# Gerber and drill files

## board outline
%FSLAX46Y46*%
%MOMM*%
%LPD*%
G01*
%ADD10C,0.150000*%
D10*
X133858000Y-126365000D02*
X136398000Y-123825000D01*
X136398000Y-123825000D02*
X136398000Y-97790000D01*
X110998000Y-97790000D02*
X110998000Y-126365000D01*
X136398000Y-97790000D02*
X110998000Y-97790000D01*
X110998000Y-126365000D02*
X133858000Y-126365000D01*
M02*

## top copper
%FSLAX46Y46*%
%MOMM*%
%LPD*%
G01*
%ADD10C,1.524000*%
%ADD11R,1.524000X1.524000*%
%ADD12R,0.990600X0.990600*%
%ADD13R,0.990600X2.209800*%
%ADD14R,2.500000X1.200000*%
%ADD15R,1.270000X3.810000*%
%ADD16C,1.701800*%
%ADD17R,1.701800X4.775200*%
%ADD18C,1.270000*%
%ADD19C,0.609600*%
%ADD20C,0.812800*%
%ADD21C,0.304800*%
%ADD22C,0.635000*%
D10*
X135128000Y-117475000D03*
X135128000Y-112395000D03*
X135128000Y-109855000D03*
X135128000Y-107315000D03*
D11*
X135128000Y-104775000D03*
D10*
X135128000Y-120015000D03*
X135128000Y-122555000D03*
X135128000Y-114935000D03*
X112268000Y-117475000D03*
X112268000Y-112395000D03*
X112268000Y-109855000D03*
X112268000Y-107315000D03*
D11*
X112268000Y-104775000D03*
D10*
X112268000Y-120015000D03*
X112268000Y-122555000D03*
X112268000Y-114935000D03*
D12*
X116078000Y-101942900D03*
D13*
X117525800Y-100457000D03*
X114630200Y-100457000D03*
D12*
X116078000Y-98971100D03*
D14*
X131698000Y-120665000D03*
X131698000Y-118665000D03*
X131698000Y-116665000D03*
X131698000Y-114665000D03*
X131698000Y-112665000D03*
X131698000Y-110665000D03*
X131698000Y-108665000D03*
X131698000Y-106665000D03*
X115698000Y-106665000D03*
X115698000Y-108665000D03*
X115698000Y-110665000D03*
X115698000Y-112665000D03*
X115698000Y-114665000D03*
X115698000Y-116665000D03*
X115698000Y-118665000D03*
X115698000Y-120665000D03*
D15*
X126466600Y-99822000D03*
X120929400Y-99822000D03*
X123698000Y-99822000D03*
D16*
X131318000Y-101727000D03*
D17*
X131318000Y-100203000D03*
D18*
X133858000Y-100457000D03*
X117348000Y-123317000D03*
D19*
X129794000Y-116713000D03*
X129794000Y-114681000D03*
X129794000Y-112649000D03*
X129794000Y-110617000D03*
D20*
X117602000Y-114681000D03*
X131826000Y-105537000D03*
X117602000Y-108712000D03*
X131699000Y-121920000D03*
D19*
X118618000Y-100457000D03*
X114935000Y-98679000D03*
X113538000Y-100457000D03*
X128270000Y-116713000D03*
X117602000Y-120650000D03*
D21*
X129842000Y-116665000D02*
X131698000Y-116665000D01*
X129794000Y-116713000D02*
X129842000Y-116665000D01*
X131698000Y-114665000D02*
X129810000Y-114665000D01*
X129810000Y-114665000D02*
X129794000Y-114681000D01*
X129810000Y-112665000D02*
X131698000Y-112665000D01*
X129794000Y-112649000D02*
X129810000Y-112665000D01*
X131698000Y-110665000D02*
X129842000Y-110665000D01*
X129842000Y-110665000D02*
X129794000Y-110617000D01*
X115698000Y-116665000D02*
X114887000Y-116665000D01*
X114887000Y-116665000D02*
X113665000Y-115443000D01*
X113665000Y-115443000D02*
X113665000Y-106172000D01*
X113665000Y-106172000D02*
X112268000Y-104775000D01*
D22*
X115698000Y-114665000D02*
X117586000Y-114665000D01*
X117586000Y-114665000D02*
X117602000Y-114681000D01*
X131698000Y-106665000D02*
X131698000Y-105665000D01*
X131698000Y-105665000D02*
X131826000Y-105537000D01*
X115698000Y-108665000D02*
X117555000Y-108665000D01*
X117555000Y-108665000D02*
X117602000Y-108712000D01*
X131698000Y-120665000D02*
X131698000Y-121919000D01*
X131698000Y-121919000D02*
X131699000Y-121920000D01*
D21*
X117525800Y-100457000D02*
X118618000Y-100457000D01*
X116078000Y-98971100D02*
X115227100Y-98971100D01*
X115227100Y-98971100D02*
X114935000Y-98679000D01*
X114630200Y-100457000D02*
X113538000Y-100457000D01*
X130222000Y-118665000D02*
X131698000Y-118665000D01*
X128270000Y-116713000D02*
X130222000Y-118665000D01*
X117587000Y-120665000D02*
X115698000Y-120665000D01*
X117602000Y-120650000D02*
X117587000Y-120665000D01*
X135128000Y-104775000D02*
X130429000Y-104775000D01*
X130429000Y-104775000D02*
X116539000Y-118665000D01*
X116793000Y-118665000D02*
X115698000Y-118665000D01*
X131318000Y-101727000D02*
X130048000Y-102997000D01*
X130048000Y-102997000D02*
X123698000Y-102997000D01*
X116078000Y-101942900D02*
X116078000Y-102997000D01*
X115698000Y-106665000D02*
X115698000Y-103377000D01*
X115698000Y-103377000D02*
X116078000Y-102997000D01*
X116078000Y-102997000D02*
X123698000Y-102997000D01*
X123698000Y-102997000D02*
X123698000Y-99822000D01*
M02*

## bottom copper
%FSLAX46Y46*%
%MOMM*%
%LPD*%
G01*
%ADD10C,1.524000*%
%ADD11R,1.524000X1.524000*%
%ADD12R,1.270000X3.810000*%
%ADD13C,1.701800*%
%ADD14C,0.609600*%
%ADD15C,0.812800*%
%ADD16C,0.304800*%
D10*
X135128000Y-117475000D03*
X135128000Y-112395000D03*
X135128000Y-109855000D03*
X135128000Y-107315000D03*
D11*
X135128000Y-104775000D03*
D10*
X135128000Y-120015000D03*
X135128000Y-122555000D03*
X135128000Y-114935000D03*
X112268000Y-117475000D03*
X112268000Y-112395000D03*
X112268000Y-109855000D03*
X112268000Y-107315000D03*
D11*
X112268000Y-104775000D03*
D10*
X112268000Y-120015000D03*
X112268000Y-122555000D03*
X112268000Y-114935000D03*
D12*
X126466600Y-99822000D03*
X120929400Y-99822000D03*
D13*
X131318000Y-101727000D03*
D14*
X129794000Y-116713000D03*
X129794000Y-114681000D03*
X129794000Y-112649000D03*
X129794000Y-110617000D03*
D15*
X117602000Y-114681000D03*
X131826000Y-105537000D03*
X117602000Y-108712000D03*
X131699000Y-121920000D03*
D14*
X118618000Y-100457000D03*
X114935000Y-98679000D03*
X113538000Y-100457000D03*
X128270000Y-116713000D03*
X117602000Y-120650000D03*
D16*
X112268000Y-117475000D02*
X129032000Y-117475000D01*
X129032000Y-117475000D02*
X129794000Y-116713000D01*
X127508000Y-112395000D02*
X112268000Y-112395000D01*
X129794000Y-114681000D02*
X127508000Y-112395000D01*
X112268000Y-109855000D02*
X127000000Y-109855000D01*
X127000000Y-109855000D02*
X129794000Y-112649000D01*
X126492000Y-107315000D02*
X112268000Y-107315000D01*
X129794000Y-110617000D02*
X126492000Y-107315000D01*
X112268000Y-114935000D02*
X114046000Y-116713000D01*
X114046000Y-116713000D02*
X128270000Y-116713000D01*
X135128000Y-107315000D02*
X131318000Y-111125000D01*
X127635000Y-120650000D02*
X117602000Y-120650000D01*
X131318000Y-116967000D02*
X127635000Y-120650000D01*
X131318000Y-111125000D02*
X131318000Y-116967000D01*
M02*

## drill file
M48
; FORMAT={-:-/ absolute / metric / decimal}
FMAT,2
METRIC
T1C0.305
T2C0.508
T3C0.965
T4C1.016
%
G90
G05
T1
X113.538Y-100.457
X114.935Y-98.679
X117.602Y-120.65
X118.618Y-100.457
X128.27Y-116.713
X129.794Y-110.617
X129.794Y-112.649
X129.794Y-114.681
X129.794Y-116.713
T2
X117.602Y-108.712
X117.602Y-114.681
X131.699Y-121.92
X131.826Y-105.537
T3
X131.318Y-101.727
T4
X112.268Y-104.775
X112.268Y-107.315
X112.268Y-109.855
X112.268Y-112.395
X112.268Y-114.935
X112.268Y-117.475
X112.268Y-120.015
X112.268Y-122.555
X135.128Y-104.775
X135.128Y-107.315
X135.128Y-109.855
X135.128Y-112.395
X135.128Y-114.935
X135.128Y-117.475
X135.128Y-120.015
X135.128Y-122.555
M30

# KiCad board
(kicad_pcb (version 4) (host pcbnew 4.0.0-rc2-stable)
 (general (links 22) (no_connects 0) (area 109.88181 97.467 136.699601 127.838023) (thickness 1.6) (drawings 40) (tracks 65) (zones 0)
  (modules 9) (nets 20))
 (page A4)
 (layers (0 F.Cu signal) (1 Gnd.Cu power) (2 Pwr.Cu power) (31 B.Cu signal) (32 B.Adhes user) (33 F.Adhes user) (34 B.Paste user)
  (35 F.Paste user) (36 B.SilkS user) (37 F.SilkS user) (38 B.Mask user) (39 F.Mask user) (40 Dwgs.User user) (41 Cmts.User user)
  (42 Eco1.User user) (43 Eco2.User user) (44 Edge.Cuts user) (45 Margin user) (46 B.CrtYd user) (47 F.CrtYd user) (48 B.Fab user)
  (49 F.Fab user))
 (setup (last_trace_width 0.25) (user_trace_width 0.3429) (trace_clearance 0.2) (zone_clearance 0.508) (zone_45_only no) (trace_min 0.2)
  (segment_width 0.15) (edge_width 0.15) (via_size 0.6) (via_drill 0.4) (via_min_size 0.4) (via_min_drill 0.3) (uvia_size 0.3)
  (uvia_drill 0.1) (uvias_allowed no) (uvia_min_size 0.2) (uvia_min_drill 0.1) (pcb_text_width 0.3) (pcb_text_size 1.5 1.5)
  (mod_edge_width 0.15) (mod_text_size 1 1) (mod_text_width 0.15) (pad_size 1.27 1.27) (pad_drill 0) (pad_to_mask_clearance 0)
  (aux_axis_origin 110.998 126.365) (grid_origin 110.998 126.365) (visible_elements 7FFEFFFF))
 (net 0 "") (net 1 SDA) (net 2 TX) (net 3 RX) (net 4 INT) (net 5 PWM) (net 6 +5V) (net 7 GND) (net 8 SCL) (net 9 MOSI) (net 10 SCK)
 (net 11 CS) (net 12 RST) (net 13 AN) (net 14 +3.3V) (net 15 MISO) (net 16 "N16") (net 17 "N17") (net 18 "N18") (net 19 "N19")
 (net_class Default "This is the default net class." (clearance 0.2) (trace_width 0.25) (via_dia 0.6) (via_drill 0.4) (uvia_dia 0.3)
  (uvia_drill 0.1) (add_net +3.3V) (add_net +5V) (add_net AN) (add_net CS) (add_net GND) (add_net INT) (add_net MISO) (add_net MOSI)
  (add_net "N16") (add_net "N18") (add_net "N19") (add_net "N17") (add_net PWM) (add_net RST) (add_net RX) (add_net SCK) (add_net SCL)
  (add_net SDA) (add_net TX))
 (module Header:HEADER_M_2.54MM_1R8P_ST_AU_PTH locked (layer B.Cu) (at 135.128 113.665 270)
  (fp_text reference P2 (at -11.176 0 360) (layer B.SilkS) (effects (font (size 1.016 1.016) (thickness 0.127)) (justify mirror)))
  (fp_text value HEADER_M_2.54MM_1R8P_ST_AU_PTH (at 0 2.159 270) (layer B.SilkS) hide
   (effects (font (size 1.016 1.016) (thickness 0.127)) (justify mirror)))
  (pad 6 thru_hole circle (at 3.81 0 270) (size 1.524 1.524) (drill 1.016) (layers *.Cu *.Mask) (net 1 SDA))
  (pad 4 thru_hole circle (at -1.27 0 270) (size 1.524 1.524) (drill 1.016) (layers *.Cu *.Mask) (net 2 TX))
  (pad 3 thru_hole circle (at -3.81 0 270) (size 1.524 1.524) (drill 1.016) (layers *.Cu *.Mask) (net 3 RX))
  (pad 2 thru_hole circle (at -6.35 0 270) (size 1.524 1.524) (drill 1.016) (layers *.Cu *.Mask) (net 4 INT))
  (pad 1 thru_hole rect (at -8.89 0 270) (size 1.524 1.524) (drill 1.016) (layers *.Cu *.Mask) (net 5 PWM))
  (pad 7 thru_hole circle (at 6.35 0 270) (size 1.524 1.524) (drill 1.016) (layers *.Cu *.Mask) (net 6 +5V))
  (pad 8 thru_hole circle (at 8.89 0 270) (size 1.524 1.524) (drill 1.016) (layers *.Cu *.Mask) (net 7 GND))
  (pad 5 thru_hole circle (at 1.27 0 270) (size 1.524 1.524) (drill 1.016) (layers *.Cu *.Mask) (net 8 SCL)))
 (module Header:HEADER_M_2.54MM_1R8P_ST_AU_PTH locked (layer B.Cu) (at 112.268 113.665 270)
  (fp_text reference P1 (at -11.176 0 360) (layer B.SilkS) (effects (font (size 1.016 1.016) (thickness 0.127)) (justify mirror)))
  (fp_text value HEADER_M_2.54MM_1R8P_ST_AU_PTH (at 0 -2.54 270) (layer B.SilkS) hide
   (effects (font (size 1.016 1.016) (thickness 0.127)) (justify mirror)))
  (pad 6 thru_hole circle (at 3.81 0 270) (size 1.524 1.524) (drill 1.016) (layers *.Cu *.Mask) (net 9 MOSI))
  (pad 4 thru_hole circle (at -1.27 0 270) (size 1.524 1.524) (drill 1.016) (layers *.Cu *.Mask) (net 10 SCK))
  (pad 3 thru_hole circle (at -3.81 0 270) (size 1.524 1.524) (drill 1.016) (layers *.Cu *.Mask) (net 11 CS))
  (pad 2 thru_hole circle (at -6.35 0 270) (size 1.524 1.524) (drill 1.016) (layers *.Cu *.Mask) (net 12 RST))
  (pad 1 thru_hole rect (at -8.89 0 270) (size 1.524 1.524) (drill 1.016) (layers *.Cu *.Mask) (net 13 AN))
  (pad 7 thru_hole circle (at 6.35 0 270) (size 1.524 1.524) (drill 1.016) (layers *.Cu *.Mask) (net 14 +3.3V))
  (pad 8 thru_hole circle (at 8.89 0 270) (size 1.524 1.524) (drill 1.016) (layers *.Cu *.Mask) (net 7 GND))
  (pad 5 thru_hole circle (at 1.27 0 270) (size 1.524 1.524) (drill 1.016) (layers *.Cu *.Mask) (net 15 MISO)))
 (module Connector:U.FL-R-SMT (layer F.Cu) (at 116.078 100.457)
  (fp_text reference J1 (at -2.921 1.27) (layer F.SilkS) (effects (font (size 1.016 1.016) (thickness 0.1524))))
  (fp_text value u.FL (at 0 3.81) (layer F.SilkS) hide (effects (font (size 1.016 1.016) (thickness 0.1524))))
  (pad 1 smd rect (at 0 1.4859) (size 0.9906 0.9906) (layers F.Cu F.Paste F.Mask) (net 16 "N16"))
  (pad 4 smd rect (at 1.4478 0) (size 0.9906 2.2098) (layers F.Cu F.Paste F.Mask) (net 7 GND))
  (pad 2 smd rect (at -1.4478 0) (size 0.9906 2.2098) (layers F.Cu F.Paste F.Mask) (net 7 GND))
  (pad 3 smd rect (at 0 -1.4859) (size 0.9906 0.9906) (layers F.Cu F.Paste F.Mask) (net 7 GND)))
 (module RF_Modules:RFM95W (layer F.Cu) (at 123.698 113.665 180)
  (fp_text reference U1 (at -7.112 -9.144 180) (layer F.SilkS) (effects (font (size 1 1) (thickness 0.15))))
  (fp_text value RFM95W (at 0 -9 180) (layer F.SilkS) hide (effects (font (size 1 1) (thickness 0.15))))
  (pad 1 smd rect (at -8 -7 180) (size 2.5 1.2) (layers F.Cu F.Paste F.Mask) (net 7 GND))
  (pad 2 smd rect (at -8 -5 180) (size 2.5 1.2) (layers F.Cu F.Paste F.Mask) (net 15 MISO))
  (pad 3 smd rect (at -8 -3 180) (size 2.5 1.2) (layers F.Cu F.Paste F.Mask) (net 9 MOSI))
  (pad 4 smd rect (at -8 -1 180) (size 2.5 1.2) (layers F.Cu F.Paste F.Mask) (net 10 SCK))
  (pad 5 smd rect (at -8 1 180) (size 2.5 1.2) (layers F.Cu F.Paste F.Mask) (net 11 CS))
  (pad 6 smd rect (at -8 3 180) (size 2.5 1.2) (layers F.Cu F.Paste F.Mask) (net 12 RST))
  (pad 7 smd rect (at -8 5 180) (size 2.5 1.2) (layers F.Cu F.Paste F.Mask) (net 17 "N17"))
  (pad 8 smd rect (at -8 7 180) (size 2.5 1.2) (layers F.Cu F.Paste F.Mask) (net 7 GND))
  (pad 9 smd rect (at 8 7 180) (size 2.5 1.2) (layers F.Cu F.Paste F.Mask) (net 16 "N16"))
  (pad 10 smd rect (at 8 5 180) (size 2.5 1.2) (layers F.Cu F.Paste F.Mask) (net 7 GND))
  (pad 11 smd rect (at 8 3 180) (size 2.5 1.2) (layers F.Cu F.Paste F.Mask) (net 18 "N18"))
  (pad 12 smd rect (at 8 1 180) (size 2.5 1.2) (layers F.Cu F.Paste F.Mask) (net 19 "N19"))
  (pad 13 smd rect (at 8 -1 180) (size 2.5 1.2) (layers F.Cu F.Paste F.Mask) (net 14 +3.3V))
  (pad 14 smd rect (at 8 -3 180) (size 2.5 1.2) (layers F.Cu F.Paste F.Mask) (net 13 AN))
  (pad 15 smd rect (at 8 -5 180) (size 2.5 1.2) (layers F.Cu F.Paste F.Mask) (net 5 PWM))
  (pad 16 smd rect (at 8 -7 180) (size 2.5 1.2) (layers F.Cu F.Paste F.Mask) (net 4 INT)))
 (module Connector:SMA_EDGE (layer F.Cu) (at 123.698 97.917 270)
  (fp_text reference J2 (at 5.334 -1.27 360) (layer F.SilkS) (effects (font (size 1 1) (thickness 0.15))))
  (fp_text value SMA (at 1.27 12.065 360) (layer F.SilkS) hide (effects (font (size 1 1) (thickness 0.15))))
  (pad 2 smd rect (at 1.905 -2.7686 270) (size 3.81 1.27) (layers *.Cu F.Paste F.Mask) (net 7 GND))
  (pad 3 smd rect (at 1.905 2.7686 270) (size 3.81 1.27) (layers *.Cu F.Paste F.Mask) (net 7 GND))
  (pad 1 smd rect (at 1.905 0 270) (size 3.81 1.27) (layers F.Cu F.Paste F.Mask) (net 16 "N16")))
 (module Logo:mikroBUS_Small (layer B.Cu) (at 123.698 104.775 180)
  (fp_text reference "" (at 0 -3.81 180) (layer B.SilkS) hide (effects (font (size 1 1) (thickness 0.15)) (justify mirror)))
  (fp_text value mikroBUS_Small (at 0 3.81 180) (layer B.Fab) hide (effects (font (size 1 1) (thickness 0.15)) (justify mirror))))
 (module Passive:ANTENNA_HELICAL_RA (layer F.Cu) (at 131.318 101.727)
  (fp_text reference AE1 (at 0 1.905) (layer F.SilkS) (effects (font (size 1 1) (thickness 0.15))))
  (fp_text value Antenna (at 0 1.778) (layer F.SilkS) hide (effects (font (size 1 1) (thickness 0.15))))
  (pad 1 thru_hole circle (at 0 0) (size 1.7018 1.7018) (drill 0.9652) (layers *.Cu *.Mask) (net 16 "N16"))
  (pad 1 smd rect (at 0 -1.524) (size 1.7018 4.7752) (layers F.Cu F.Mask) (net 16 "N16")))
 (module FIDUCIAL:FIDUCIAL (layer F.Cu) (at 133.858 100.457)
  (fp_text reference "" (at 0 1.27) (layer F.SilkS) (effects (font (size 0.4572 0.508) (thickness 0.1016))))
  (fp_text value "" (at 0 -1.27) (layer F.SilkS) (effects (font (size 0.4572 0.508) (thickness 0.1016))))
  (pad 1 smd circle (at 0 0 270) (size 1.27 1.27) (layers F.Cu F.Mask) (solder_mask_margin 0.635) (clearance 0.635)))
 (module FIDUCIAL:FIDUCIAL (layer F.Cu) (at 117.348 123.317)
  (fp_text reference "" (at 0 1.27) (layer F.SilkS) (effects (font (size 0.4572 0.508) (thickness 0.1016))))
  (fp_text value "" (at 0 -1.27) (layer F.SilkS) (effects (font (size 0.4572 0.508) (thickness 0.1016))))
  (pad 1 smd circle (at 0 0 270) (size 1.27 1.27) (layers F.Cu F.Mask) (solder_mask_margin 0.635) (clearance 0.635)))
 (gr_line (start 133.858 126.365) (end 136.398 123.825) (angle 90) (layer Edge.Cuts) (width 0.15))
 (gr_line (start 136.398 123.825) (end 136.398 97.79) (angle 90) (layer Edge.Cuts) (width 0.15))
 (gr_line (start 110.998 97.79) (end 110.998 126.365) (angle 90) (layer Edge.Cuts) (width 0.15))
 (gr_line (start 136.398 97.79) (end 110.998 97.79) (angle 90) (layer Edge.Cuts) (width 0.15))
 (gr_line (start 110.998 126.365) (end 133.858 126.365) (angle 90) (layer Edge.Cuts) (width 0.15))
 (segment (start 112.268 117.475) (end 129.032 117.475) (width 0.3048) (layer B.Cu) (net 9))
 (segment (start 129.842 116.665) (end 131.698 116.665) (width 0.3048) (layer F.Cu) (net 9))
 (segment (start 129.794 116.713) (end 129.842 116.665) (width 0.3048) (layer F.Cu) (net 9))
 (via (at 129.794 116.713) (size 0.6096) (drill 0.3048) (layers F.Cu B.Cu) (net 9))
 (segment (start 129.032 117.475) (end 129.794 116.713) (width 0.3048) (layer B.Cu) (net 9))
 (segment (start 131.698 114.665) (end 129.81 114.665) (width 0.3048) (layer F.Cu) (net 10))
 (segment (start 127.508 112.395) (end 112.268 112.395) (width 0.3048) (layer B.Cu) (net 10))
 (segment (start 129.794 114.681) (end 127.508 112.395) (width 0.3048) (layer B.Cu) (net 10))
 (via (at 129.794 114.681) (size 0.6096) (drill 0.3048) (layers F.Cu B.Cu) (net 10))
 (segment (start 129.81 114.665) (end 129.794 114.681) (width 0.3048) (layer F.Cu) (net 10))
 (segment (start 112.268 109.855) (end 127 109.855) (width 0.3048) (layer B.Cu) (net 11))
 (segment (start 129.81 112.665) (end 131.698 112.665) (width 0.3048) (layer F.Cu) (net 11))
 (segment (start 129.794 112.649) (end 129.81 112.665) (width 0.3048) (layer F.Cu) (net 11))
 (via (at 129.794 112.649) (size 0.6096) (drill 0.3048) (layers F.Cu B.Cu) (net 11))
 (segment (start 127 109.855) (end 129.794 112.649) (width 0.3048) (layer B.Cu) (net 11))
 (segment (start 131.698 110.665) (end 129.842 110.665) (width 0.3048) (layer F.Cu) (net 12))
 (segment (start 126.492 107.315) (end 112.268 107.315) (width 0.3048) (layer B.Cu) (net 12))
 (segment (start 129.794 110.617) (end 126.492 107.315) (width 0.3048) (layer B.Cu) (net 12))
 (via (at 129.794 110.617) (size 0.6096) (drill 0.3048) (layers F.Cu B.Cu) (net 12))
 (segment (start 129.842 110.665) (end 129.794 110.617) (width 0.3048) (layer F.Cu) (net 12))
 (segment (start 115.698 116.665) (end 114.887 116.665) (width 0.3048) (layer F.Cu) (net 13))
 (segment (start 114.887 116.665) (end 113.665 115.443) (width 0.3048) (layer F.Cu) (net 13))
 (segment (start 113.665 115.443) (end 113.665 106.172) (width 0.3048) (layer F.Cu) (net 13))
 (segment (start 113.665 106.172) (end 112.268 104.775) (width 0.3048) (layer F.Cu) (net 13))
 (segment (start 115.698 114.665) (end 117.586 114.665) (width 0.635) (layer F.Cu) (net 14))
 (via (at 117.602 114.681) (size 0.8128) (drill 0.508) (layers F.Cu B.Cu) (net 14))
 (segment (start 117.586 114.665) (end 117.602 114.681) (width 0.635) (layer F.Cu) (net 14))
 (segment (start 131.698 106.665) (end 131.698 105.665) (width 0.635) (layer F.Cu) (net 7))
 (via (at 131.826 105.537) (size 0.8128) (drill 0.508) (layers F.Cu B.Cu) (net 7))
 (segment (start 131.698 105.665) (end 131.826 105.537) (width 0.635) (layer F.Cu) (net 7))
 (segment (start 115.698 108.665) (end 117.555 108.665) (width 0.635) (layer F.Cu) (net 7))
 (via (at 117.602 108.712) (size 0.8128) (drill 0.508) (layers F.Cu B.Cu) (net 7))
 (segment (start 117.555 108.665) (end 117.602 108.712) (width 0.635) (layer F.Cu) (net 7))
 (segment (start 131.698 120.665) (end 131.698 121.919) (width 0.635) (layer F.Cu) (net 7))
 (via (at 131.699 121.92) (size 0.8128) (drill 0.508) (layers F.Cu B.Cu) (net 7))
 (segment (start 131.698 121.919) (end 131.699 121.92) (width 0.635) (layer F.Cu) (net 7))
 (segment (start 117.5258 100.457) (end 118.618 100.457) (width 0.3048) (layer F.Cu) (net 7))
 (via (at 118.618 100.457) (size 0.6096) (drill 0.3048) (layers F.Cu B.Cu) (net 7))
 (segment (start 116.078 98.9711) (end 115.2271 98.9711) (width 0.3048) (layer F.Cu) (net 7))
 (via (at 114.935 98.679) (size 0.6096) (drill 0.3048) (layers F.Cu B.Cu) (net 7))
 (segment (start 115.2271 98.9711) (end 114.935 98.679) (width 0.3048) (layer F.Cu) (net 7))
 (segment (start 114.6302 100.457) (end 113.538 100.457) (width 0.3048) (layer F.Cu) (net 7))
 (via (at 113.538 100.457) (size 0.6096) (drill 0.3048) (layers F.Cu B.Cu) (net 7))
 (segment (start 112.268 114.935) (end 114.046 116.713) (width 0.3048) (layer B.Cu) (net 15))
 (segment (start 130.222 118.665) (end 131.698 118.665) (width 0.3048) (layer F.Cu) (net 15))
 (segment (start 128.27 116.713) (end 130.222 118.665) (width 0.3048) (layer F.Cu) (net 15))
 (via (at 128.27 116.713) (size 0.6096) (drill 0.3048) (layers F.Cu B.Cu) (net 15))
 (segment (start 114.046 116.713) (end 128.27 116.713) (width 0.3048) (layer B.Cu) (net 15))
 (segment (start 135.128 107.315) (end 131.318 111.125) (width 0.3048) (layer B.Cu) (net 4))
 (segment (start 117.587 120.665) (end 115.698 120.665) (width 0.3048) (layer F.Cu) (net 4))
 (segment (start 117.602 120.65) (end 117.587 120.665) (width 0.3048) (layer F.Cu) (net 4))
 (via (at 117.602 120.65) (size 0.6096) (drill 0.3048) (layers F.Cu B.Cu) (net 4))
 (segment (start 127.635 120.65) (end 117.602 120.65) (width 0.3048) (layer B.Cu) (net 4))
 (segment (start 131.318 116.967) (end 127.635 120.65) (width 0.3048) (layer B.Cu) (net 4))
 (segment (start 131.318 111.125) (end 131.318 116.967) (width 0.3048) (layer B.Cu) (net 4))
 (segment (start 135.128 104.775) (end 130.429 104.775) (width 0.3048) (layer F.Cu) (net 5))
 (segment (start 130.429 104.775) (end 116.539 118.665) (width 0.3048) (layer F.Cu) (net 5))
 (segment (start 116.793 118.665) (end 115.698 118.665) (width 0.3048) (layer F.Cu) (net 5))
 (segment (start 131.318 101.727) (end 130.048 102.997) (width 0.3048) (layer F.Cu) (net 16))
 (segment (start 130.048 102.997) (end 123.698 102.997) (width 0.3048) (layer F.Cu) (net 16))
 (segment (start 116.078 101.9429) (end 116.078 102.997) (width 0.3048) (layer F.Cu) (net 16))
 (segment (start 115.698 106.665) (end 115.698 103.377) (width 0.3048) (layer F.Cu) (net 16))
 (segment (start 115.698 103.377) (end 116.078 102.997) (width 0.3048) (layer F.Cu) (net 16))
 (segment (start 116.078 102.997) (end 123.698 102.997) (width 0.3048) (layer F.Cu) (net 16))
 (segment (start 123.698 102.997) (end 123.698 99.822) (width 0.3048) (layer F.Cu) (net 16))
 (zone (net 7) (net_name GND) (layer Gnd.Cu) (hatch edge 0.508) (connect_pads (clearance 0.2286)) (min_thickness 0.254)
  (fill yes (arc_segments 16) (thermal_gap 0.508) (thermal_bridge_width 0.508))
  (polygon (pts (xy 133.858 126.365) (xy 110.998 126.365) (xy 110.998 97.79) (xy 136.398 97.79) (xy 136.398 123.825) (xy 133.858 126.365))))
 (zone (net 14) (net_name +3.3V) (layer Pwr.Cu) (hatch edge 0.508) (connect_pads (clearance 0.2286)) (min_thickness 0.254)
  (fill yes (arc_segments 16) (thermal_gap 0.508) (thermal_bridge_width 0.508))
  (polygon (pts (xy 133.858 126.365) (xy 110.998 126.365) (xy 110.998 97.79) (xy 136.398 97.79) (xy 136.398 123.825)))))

